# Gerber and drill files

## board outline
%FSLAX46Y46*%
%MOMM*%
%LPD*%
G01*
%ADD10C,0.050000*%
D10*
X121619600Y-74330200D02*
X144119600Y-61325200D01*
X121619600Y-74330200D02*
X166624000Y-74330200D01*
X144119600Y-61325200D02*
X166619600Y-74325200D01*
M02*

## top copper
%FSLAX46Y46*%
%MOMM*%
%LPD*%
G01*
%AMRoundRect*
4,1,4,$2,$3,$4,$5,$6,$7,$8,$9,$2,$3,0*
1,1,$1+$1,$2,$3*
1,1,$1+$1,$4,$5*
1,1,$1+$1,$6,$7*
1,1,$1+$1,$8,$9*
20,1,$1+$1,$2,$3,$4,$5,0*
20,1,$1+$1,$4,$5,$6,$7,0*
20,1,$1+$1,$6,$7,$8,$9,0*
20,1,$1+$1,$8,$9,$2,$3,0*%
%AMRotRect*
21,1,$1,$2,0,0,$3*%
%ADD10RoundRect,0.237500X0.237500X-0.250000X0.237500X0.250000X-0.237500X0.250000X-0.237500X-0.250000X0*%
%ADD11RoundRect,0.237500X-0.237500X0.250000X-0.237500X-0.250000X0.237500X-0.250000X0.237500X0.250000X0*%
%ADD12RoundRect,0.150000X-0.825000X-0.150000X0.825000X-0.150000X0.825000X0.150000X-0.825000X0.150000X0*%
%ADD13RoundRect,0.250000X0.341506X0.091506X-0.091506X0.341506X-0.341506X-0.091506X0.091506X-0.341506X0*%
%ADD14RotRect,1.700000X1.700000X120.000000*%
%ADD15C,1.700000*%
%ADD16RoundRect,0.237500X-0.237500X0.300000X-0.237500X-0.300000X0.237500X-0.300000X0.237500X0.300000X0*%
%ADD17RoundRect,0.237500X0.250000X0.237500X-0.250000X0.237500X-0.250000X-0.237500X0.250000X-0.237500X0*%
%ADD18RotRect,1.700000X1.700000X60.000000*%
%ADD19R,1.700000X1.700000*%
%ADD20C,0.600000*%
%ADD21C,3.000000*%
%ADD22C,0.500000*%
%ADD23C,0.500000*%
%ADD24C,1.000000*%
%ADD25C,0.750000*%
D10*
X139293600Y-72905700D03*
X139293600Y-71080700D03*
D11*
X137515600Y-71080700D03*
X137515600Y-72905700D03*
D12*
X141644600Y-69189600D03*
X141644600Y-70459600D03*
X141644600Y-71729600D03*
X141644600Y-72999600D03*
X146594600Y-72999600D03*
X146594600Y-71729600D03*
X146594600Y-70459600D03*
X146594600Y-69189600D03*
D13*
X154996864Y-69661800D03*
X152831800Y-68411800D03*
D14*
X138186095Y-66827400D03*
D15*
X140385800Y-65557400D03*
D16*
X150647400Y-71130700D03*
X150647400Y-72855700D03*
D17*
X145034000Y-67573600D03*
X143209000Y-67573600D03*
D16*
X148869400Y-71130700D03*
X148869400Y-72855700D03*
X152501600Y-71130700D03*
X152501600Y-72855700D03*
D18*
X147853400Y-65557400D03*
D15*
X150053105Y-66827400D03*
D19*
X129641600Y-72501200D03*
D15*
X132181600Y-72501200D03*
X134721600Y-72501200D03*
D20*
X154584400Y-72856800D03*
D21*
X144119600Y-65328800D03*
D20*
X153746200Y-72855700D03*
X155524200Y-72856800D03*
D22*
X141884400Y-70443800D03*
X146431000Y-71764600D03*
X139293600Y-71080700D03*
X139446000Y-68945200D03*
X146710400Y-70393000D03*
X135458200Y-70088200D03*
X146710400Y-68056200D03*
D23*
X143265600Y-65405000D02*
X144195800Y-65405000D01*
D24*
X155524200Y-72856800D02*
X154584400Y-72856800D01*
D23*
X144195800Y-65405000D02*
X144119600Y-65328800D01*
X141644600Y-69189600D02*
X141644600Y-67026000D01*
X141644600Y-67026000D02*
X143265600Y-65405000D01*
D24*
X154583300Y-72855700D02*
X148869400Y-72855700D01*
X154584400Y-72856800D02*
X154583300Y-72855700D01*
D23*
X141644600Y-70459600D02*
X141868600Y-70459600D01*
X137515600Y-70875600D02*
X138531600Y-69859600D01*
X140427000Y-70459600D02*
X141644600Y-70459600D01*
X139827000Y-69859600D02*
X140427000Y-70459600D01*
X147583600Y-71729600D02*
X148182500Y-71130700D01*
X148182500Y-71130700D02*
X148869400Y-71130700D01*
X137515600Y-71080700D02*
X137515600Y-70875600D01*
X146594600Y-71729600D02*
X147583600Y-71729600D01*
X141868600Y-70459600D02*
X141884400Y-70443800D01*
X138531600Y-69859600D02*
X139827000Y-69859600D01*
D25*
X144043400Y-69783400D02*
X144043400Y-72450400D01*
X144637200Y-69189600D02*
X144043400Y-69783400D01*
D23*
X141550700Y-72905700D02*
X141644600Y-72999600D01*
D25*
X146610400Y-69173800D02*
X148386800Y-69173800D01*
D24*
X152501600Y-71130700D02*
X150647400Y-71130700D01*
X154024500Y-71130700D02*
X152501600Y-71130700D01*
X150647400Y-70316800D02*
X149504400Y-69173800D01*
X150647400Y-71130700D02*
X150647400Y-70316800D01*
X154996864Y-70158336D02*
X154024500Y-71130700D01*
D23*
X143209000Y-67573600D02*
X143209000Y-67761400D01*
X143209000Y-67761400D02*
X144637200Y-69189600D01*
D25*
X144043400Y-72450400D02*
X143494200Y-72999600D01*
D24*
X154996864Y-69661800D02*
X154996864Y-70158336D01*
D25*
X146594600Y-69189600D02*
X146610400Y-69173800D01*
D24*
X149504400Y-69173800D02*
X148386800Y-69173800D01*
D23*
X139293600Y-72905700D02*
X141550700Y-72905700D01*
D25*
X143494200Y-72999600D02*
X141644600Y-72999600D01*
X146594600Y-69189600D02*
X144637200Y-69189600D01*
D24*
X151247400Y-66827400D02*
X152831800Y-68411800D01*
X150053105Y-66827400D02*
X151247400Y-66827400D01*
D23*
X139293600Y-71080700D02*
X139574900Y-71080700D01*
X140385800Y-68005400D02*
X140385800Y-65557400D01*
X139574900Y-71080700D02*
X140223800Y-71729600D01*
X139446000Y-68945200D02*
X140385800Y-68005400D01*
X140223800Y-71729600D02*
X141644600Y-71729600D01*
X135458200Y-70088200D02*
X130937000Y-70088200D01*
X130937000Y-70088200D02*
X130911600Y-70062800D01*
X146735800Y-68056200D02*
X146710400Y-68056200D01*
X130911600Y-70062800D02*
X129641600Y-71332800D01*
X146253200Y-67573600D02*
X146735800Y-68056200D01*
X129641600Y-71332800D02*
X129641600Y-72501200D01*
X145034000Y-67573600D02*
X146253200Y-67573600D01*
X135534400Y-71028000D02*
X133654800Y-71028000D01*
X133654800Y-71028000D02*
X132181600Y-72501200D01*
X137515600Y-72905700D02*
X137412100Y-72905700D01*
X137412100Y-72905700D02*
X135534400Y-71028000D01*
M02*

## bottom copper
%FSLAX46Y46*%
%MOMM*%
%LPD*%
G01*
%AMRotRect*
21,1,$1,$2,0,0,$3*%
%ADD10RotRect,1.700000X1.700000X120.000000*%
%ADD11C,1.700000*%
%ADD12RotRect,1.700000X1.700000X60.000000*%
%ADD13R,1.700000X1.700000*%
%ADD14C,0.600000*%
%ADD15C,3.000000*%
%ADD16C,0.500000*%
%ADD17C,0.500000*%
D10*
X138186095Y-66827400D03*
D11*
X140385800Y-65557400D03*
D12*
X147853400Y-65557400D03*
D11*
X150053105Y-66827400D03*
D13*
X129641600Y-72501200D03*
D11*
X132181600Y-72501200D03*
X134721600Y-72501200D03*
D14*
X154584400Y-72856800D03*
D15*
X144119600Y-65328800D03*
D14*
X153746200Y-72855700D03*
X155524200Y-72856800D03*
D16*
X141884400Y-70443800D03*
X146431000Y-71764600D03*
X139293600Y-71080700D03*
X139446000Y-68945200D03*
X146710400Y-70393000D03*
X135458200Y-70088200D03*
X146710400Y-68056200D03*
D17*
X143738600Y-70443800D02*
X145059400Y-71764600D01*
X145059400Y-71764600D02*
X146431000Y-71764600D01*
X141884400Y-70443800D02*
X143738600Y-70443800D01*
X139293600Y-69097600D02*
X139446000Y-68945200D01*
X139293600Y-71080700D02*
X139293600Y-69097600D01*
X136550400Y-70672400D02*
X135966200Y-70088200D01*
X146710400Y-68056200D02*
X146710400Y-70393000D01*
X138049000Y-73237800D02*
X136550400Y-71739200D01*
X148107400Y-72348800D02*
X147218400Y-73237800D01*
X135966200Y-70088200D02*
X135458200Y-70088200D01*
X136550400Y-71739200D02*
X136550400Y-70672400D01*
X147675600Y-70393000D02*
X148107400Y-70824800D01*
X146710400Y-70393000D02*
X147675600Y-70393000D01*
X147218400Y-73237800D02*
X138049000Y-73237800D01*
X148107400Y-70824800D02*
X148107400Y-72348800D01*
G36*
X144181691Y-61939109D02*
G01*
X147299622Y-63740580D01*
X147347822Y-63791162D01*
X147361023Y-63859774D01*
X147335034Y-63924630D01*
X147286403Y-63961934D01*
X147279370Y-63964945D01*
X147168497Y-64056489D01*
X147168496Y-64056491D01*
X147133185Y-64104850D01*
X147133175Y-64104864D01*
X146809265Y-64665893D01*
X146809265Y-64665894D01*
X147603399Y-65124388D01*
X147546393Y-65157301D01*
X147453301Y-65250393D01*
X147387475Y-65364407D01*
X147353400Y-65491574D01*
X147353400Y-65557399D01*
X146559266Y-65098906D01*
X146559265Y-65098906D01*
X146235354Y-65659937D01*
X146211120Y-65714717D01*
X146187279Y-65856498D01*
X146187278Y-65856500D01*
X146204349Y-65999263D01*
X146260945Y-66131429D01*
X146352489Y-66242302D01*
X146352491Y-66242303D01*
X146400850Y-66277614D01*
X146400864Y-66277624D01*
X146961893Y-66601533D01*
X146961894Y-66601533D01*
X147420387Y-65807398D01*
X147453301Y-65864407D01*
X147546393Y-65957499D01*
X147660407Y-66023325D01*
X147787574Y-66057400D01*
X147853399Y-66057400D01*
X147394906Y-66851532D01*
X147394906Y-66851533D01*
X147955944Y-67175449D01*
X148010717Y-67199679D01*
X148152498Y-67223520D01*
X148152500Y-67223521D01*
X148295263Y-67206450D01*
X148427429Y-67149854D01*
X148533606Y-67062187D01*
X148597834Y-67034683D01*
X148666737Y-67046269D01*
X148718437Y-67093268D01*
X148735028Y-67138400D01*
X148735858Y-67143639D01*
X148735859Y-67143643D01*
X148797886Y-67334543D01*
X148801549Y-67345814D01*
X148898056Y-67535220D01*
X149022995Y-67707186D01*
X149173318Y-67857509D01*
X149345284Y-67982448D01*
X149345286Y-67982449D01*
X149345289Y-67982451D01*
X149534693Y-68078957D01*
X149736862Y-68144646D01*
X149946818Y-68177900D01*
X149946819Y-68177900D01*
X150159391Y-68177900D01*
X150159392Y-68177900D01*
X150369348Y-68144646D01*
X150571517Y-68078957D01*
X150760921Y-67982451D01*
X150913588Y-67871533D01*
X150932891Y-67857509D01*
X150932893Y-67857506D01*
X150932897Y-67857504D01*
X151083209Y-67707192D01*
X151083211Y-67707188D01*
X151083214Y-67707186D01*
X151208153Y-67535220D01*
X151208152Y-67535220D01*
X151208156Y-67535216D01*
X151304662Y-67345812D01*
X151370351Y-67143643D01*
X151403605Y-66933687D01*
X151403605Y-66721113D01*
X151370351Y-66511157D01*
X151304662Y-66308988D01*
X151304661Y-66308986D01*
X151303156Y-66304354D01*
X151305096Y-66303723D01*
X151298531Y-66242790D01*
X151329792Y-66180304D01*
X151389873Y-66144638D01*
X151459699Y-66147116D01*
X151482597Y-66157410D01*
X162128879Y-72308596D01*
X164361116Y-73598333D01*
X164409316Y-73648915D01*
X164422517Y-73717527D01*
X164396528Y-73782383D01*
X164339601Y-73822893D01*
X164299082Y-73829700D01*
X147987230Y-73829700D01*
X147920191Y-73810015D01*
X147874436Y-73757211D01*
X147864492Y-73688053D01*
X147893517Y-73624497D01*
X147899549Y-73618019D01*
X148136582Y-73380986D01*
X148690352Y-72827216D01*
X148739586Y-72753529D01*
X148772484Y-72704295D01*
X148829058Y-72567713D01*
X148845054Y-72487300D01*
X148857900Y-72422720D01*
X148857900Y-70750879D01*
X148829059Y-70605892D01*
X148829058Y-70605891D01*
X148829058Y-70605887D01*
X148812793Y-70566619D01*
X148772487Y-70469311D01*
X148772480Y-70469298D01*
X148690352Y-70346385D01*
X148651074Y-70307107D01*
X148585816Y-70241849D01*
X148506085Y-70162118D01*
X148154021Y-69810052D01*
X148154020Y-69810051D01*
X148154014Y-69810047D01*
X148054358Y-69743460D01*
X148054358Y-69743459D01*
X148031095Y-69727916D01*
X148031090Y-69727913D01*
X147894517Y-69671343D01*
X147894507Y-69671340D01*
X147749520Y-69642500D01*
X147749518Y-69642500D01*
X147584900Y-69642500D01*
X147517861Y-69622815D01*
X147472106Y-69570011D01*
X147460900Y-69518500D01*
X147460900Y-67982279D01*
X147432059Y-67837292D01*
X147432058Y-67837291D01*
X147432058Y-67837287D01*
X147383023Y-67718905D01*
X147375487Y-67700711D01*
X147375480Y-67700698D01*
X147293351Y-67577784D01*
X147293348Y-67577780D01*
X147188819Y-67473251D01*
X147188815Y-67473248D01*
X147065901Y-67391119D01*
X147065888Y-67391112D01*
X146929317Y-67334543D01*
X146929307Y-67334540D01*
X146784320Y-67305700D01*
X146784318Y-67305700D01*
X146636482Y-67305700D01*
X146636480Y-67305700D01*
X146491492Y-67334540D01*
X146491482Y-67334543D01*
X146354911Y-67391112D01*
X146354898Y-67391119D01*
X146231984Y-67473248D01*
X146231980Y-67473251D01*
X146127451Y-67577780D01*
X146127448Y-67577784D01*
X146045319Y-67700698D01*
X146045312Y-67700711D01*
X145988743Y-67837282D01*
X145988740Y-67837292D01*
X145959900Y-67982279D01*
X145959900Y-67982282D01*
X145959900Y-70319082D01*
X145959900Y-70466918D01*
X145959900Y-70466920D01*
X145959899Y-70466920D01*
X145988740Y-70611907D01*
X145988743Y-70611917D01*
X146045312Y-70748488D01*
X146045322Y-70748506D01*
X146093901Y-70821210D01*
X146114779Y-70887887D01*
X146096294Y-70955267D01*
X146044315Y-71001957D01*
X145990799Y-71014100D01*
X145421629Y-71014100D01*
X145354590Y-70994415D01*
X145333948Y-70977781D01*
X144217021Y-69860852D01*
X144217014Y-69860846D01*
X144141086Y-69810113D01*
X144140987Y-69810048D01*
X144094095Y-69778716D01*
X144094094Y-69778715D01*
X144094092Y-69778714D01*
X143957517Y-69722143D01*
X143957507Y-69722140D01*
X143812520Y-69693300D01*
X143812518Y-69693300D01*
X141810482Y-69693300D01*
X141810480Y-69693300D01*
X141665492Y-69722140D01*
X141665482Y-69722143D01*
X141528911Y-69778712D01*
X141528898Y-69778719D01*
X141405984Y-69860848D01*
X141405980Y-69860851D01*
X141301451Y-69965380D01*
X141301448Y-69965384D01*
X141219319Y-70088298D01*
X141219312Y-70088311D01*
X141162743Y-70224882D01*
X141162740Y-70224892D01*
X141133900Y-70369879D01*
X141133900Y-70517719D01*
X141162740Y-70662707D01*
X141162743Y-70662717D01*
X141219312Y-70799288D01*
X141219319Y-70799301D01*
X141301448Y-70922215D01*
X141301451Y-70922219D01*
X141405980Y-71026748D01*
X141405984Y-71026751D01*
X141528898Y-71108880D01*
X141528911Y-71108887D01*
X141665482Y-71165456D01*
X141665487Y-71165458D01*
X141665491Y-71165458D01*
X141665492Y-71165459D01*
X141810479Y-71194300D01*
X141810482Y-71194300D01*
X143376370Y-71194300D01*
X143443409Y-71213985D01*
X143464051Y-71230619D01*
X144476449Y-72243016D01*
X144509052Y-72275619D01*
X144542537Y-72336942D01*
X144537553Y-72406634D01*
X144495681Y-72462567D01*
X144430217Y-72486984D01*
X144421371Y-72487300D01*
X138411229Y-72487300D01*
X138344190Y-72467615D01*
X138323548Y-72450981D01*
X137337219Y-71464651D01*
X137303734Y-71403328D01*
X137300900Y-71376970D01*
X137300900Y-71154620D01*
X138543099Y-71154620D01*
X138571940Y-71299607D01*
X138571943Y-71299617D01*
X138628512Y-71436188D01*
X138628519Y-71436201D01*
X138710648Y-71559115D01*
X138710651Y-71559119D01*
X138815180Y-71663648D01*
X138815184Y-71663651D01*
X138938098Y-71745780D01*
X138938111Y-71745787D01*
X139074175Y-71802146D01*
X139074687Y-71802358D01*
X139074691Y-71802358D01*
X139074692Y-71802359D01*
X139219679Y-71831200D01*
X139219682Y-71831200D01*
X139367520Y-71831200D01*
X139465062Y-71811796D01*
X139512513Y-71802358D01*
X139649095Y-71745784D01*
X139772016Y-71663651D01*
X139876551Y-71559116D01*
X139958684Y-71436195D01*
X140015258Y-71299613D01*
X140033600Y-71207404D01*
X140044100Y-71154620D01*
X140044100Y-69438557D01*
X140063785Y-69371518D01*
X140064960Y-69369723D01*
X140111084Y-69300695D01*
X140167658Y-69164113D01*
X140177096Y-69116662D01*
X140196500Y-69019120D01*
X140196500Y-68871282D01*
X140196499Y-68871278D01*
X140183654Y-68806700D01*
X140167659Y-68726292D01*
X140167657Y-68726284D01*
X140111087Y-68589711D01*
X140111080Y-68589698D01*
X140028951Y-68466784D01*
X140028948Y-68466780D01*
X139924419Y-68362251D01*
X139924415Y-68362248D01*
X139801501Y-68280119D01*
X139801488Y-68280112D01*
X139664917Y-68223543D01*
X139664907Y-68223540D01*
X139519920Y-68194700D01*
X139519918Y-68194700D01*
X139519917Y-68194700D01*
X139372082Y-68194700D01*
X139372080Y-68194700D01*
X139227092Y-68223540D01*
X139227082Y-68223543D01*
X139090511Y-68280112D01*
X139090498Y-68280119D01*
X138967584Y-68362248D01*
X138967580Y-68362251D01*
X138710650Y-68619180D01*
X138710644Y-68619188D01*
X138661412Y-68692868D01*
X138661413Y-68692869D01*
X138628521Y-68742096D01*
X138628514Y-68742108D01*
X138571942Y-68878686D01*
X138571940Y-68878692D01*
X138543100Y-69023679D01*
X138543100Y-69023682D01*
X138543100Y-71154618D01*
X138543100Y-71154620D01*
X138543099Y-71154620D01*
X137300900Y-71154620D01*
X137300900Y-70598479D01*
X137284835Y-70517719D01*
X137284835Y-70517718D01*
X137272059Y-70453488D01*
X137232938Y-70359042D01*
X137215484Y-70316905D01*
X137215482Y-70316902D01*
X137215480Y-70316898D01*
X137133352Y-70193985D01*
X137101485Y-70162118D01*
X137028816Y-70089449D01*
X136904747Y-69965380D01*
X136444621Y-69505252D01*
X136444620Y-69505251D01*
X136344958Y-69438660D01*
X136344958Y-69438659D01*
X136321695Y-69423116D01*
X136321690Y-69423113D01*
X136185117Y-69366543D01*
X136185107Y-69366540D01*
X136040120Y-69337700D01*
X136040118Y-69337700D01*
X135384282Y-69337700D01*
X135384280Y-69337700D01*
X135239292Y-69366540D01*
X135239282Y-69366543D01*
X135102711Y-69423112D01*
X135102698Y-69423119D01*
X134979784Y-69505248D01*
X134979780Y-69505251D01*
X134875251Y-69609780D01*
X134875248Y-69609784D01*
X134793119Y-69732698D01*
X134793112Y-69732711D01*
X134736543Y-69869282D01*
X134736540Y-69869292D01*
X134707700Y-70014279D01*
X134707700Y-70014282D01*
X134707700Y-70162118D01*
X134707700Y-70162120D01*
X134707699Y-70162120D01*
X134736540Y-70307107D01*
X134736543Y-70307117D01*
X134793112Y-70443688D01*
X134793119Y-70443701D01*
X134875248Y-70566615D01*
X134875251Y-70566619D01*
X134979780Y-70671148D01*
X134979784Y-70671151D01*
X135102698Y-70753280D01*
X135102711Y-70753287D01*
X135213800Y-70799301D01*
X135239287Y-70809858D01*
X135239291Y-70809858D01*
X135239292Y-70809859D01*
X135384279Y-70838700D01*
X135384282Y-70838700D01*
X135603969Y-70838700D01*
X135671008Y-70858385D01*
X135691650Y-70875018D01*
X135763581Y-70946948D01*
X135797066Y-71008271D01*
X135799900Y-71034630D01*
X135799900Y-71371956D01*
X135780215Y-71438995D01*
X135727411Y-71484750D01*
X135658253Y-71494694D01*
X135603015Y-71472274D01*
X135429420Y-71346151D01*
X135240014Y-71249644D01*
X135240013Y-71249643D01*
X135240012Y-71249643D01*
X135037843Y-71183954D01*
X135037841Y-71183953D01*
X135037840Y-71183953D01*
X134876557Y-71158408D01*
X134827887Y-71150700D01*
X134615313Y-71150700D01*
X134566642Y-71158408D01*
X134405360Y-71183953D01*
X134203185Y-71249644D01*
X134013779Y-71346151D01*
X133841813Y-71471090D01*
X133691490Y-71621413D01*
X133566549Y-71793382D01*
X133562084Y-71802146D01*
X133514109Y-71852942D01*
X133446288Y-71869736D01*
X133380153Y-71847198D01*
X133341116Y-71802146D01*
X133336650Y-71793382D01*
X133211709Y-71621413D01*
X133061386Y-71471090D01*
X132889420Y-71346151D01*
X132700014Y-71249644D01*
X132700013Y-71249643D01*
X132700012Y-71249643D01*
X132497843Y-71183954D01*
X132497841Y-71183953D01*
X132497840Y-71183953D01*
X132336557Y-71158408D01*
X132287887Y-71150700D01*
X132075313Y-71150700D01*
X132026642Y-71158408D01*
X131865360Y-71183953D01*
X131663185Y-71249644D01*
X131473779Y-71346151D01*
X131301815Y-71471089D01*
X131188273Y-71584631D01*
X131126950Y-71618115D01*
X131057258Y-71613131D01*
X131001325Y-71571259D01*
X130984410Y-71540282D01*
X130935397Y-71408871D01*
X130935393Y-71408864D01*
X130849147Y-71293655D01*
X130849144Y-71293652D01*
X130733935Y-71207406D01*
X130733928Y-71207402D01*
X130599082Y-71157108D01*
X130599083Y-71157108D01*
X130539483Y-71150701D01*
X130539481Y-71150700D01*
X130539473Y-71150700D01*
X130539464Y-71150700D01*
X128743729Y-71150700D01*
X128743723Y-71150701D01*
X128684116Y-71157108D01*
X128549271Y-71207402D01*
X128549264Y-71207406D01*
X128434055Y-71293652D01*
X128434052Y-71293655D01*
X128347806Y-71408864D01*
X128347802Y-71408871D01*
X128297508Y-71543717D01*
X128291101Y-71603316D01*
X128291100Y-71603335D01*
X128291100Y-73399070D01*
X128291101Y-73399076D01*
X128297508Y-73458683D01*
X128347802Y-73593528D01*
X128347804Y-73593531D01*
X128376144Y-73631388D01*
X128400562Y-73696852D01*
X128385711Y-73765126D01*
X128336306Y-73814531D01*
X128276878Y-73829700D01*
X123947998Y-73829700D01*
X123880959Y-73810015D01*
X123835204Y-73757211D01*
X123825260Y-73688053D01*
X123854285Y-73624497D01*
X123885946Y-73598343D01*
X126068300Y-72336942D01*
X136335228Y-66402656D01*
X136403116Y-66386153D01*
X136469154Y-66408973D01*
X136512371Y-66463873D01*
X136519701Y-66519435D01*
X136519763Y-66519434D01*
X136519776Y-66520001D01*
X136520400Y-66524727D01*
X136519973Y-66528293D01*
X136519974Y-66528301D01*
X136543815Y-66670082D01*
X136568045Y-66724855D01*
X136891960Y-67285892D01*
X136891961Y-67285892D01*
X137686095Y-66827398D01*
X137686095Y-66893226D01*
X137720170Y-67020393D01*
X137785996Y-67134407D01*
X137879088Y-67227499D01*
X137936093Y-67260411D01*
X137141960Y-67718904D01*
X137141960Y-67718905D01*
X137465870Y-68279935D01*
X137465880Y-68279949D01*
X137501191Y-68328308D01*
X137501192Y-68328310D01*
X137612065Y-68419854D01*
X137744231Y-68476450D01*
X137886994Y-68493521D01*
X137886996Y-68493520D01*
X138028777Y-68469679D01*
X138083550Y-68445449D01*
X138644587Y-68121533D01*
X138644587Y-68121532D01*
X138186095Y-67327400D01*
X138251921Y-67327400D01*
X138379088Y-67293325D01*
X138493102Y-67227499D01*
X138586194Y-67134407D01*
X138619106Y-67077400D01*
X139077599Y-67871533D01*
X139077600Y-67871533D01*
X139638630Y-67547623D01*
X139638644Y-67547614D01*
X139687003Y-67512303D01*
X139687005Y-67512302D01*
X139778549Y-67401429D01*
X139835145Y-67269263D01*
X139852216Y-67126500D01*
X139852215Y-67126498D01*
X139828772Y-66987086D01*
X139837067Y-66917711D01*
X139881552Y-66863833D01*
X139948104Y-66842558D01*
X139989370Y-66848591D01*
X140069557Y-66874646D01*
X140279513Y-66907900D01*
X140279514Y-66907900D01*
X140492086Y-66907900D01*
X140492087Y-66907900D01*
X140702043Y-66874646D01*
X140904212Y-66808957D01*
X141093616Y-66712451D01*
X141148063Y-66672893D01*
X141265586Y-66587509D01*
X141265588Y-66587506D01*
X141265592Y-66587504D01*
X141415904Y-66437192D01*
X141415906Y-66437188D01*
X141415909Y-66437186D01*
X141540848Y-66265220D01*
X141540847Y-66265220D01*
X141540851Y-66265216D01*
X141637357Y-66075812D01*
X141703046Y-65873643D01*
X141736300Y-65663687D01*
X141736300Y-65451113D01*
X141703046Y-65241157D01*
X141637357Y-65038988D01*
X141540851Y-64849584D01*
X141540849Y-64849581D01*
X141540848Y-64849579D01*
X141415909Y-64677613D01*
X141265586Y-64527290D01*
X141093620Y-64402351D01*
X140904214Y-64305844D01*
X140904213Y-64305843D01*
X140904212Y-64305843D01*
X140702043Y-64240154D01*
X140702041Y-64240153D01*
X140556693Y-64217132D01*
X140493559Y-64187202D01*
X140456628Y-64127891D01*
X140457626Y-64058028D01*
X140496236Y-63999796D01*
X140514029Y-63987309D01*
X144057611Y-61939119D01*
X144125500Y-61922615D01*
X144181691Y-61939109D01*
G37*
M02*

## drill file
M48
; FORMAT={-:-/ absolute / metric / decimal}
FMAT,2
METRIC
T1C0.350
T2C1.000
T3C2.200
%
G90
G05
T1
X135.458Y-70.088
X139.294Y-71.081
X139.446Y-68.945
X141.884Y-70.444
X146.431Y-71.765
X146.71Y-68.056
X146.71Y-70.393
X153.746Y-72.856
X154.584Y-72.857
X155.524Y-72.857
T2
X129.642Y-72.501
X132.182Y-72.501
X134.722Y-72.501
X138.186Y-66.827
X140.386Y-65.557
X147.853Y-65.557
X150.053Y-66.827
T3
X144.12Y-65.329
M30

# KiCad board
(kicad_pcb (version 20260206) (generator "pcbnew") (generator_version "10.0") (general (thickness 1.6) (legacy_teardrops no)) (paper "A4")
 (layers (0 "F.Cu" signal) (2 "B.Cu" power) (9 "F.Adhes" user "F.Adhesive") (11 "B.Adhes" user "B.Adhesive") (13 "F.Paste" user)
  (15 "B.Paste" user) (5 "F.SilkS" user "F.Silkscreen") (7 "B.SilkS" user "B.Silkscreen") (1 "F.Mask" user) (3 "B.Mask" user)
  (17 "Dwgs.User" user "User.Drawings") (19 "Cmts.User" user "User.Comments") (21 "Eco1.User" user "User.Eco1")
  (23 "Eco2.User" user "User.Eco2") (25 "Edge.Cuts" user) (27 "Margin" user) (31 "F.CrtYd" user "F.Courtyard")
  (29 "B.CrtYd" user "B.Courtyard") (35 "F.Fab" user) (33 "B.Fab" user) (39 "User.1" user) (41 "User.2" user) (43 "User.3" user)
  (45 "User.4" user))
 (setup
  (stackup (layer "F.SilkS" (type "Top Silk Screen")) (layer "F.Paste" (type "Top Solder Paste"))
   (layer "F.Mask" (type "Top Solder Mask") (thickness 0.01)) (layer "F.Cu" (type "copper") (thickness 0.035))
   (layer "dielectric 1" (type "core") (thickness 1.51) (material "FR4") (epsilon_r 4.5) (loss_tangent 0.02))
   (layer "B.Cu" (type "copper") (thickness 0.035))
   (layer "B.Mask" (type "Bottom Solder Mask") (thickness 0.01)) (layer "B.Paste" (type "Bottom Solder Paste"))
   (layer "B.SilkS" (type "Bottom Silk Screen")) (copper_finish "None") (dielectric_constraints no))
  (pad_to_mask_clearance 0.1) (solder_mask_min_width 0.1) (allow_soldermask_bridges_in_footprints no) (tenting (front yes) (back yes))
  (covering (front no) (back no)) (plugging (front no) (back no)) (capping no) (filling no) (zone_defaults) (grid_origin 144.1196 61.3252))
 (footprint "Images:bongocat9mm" (layer "F.Cu") (at 158.0388 72.806)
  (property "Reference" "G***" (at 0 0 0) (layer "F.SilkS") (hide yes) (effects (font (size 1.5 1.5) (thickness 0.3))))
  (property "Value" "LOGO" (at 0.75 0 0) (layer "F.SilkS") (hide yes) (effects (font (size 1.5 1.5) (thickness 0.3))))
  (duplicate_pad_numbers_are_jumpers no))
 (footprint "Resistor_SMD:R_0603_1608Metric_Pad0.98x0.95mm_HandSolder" (layer "F.Cu") (at 139.2936 71.9932 90)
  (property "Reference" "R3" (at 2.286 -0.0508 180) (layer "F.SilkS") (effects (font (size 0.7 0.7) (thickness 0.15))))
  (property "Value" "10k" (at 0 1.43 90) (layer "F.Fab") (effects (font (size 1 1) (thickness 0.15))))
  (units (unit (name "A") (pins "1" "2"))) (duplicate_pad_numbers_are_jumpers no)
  (pad "1" smd roundrect (at -0.9125 0 90) (size 0.975 0.95) (layers "F.Cu" "F.Mask" "F.Paste") (roundrect_rratio 0.25) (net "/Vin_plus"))
  (pad "2" smd roundrect (at 0.9125 0 90) (size 0.975 0.95) (layers "F.Cu" "F.Mask" "F.Paste") (roundrect_rratio 0.25) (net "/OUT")))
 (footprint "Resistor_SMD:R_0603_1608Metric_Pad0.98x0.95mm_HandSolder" (layer "F.Cu") (at 137.5156 71.9932 -90)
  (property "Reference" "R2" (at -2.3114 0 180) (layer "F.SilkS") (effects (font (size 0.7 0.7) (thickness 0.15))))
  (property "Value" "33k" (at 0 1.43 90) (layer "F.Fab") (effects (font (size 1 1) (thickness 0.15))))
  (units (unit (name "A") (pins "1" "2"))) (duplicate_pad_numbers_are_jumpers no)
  (pad "1" smd roundrect (at -0.9125 0 270) (size 0.975 0.95) (layers "F.Cu" "F.Mask" "F.Paste") (roundrect_rratio 0.25)
   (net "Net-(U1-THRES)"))
  (pad "2" smd roundrect (at 0.9125 0 270) (size 0.975 0.95) (layers "F.Cu" "F.Mask" "F.Paste") (roundrect_rratio 0.25)
   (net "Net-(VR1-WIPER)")))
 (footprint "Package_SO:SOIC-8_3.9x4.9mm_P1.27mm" (layer "F.Cu") (at 144.1196 71.0946)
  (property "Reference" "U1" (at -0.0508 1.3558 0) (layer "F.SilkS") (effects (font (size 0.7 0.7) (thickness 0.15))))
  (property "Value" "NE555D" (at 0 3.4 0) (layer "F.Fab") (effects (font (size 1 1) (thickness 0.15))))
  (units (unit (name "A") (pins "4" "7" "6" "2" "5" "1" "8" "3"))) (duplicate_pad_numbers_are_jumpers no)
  (pad "1" smd roundrect (at -2.475 -1.905) (size 1.95 0.6) (layers "F.Cu" "F.Mask" "F.Paste") (roundrect_rratio 0.25) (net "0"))
  (pad "2" smd roundrect (at -2.475 -0.635) (size 1.95 0.6) (layers "F.Cu" "F.Mask" "F.Paste") (roundrect_rratio 0.25)
   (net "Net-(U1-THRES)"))
  (pad "3" smd roundrect (at -2.475 0.635) (size 1.95 0.6) (layers "F.Cu" "F.Mask" "F.Paste") (roundrect_rratio 0.25) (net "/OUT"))
  (pad "4" smd roundrect (at -2.475 1.905) (size 1.95 0.6) (layers "F.Cu" "F.Mask" "F.Paste") (roundrect_rratio 0.25) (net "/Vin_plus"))
  (pad "5" smd roundrect (at 2.475 1.905) (size 1.95 0.6) (layers "F.Cu" "F.Mask" "F.Paste") (roundrect_rratio 0.25)
   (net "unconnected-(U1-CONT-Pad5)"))
  (pad "6" smd roundrect (at 2.475 0.635) (size 1.95 0.6) (layers "F.Cu" "F.Mask" "F.Paste") (roundrect_rratio 0.25) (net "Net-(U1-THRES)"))
  (pad "7" smd roundrect (at 2.475 -0.635) (size 1.95 0.6) (layers "F.Cu" "F.Mask" "F.Paste") (roundrect_rratio 0.25) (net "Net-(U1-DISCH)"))
  (pad "8" smd roundrect (at 2.475 -1.905) (size 1.95 0.6) (layers "F.Cu" "F.Mask" "F.Paste") (roundrect_rratio 0.25) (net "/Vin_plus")))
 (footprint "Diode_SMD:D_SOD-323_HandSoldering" (layer "F.Cu") (at 153.914332 69.0368 150)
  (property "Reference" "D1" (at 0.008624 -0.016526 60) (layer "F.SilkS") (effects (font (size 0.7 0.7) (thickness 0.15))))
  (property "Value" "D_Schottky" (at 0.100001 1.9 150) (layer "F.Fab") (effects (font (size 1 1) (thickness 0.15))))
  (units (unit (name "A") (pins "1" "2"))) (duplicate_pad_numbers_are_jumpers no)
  (pad "1" smd roundrect (at -1.25 0 150) (size 1 1) (layers "F.Cu" "F.Mask" "F.Paste") (roundrect_rratio 0.25) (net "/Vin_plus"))
  (pad "2" smd roundrect (at 1.25 0 150) (size 1 1) (layers "F.Cu" "F.Mask" "F.Paste") (roundrect_rratio 0.25) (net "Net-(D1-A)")))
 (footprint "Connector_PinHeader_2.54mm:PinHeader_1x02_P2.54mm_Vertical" (layer "F.Cu") (at 138.186095 66.8274 120)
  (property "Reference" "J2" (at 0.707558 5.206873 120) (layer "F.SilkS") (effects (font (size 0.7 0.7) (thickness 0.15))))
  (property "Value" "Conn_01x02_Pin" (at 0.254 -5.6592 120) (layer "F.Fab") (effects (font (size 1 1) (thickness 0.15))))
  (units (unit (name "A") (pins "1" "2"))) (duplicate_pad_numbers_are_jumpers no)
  (pad "1" thru_hole rect (at 0 0 120) (size 1.7 1.7) (drill 1) (layers "*.Cu" "*.Mask") (remove_unused_layers no) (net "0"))
  (pad "2" thru_hole circle (at 0 2.54 120) (size 1.7 1.7) (drill 1) (layers "*.Cu" "*.Mask") (remove_unused_layers no) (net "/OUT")))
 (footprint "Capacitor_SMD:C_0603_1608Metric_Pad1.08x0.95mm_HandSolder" (layer "F.Cu") (at 150.6474 71.9932 -90)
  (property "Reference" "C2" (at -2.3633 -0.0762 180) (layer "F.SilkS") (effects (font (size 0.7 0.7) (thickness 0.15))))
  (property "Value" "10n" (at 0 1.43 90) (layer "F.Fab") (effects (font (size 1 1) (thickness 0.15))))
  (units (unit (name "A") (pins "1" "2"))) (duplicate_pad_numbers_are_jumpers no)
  (pad "1" smd roundrect (at -0.8625 0 270) (size 1.075 0.95) (layers "F.Cu" "F.Mask" "F.Paste") (roundrect_rratio 0.25) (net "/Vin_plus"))
  (pad "2" smd roundrect (at 0.8625 0 270) (size 1.075 0.95) (layers "F.Cu" "F.Mask" "F.Paste") (roundrect_rratio 0.25) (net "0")))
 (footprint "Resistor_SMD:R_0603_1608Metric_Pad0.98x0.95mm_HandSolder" (layer "F.Cu") (at 144.1215 67.5736 180)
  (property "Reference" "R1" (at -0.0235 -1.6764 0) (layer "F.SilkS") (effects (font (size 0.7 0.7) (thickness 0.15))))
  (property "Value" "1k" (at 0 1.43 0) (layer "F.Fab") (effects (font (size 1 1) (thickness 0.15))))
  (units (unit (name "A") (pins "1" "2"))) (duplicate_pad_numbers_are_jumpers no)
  (pad "1" smd roundrect (at -0.9125 0 180) (size 0.975 0.95) (layers "F.Cu" "F.Mask" "F.Paste") (roundrect_rratio 0.25)
   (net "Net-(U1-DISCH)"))
  (pad "2" smd roundrect (at 0.9125 0 180) (size 0.975 0.95) (layers "F.Cu" "F.Mask" "F.Paste") (roundrect_rratio 0.25) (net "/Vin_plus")))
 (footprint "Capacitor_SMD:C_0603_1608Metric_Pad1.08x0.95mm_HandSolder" (layer "F.Cu") (at 148.8694 71.9932 -90)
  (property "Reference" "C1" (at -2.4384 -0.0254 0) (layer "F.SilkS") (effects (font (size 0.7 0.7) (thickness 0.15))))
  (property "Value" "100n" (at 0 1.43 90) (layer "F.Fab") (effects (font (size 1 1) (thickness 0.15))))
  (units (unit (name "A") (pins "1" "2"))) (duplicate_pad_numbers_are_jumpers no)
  (pad "1" smd roundrect (at -0.8625 0 270) (size 1.075 0.95) (layers "F.Cu" "F.Mask" "F.Paste") (roundrect_rratio 0.25)
   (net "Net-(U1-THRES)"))
  (pad "2" smd roundrect (at 0.8625 0 270) (size 1.075 0.95) (layers "F.Cu" "F.Mask" "F.Paste") (roundrect_rratio 0.25) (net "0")))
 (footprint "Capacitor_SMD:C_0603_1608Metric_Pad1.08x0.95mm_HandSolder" (layer "F.Cu") (at 152.5016 71.9932 -90)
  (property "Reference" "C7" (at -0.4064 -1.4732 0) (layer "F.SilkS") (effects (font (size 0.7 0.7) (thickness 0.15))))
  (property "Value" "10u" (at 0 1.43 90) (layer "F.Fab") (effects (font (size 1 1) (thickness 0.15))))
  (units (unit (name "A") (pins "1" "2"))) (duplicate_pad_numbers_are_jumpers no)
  (pad "1" smd roundrect (at -0.8625 0 270) (size 1.075 0.95) (layers "F.Cu" "F.Mask" "F.Paste") (roundrect_rratio 0.25) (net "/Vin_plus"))
  (pad "2" smd roundrect (at 0.8625 0 270) (size 1.075 0.95) (layers "F.Cu" "F.Mask" "F.Paste") (roundrect_rratio 0.25) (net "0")))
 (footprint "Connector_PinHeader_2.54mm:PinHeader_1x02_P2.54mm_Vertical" (layer "F.Cu") (at 147.8534 65.5574 60)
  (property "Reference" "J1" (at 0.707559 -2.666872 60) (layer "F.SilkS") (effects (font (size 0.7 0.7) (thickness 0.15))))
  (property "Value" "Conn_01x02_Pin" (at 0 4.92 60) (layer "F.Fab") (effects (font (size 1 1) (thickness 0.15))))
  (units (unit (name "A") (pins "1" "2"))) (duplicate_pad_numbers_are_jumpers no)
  (pad "1" thru_hole rect (at 0 0 60) (size 1.7 1.7) (drill 1) (layers "*.Cu" "*.Mask") (remove_unused_layers no) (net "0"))
  (pad "2" thru_hole circle (at 0 2.54 60) (size 1.7 1.7) (drill 1) (layers "*.Cu" "*.Mask") (remove_unused_layers no) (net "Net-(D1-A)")))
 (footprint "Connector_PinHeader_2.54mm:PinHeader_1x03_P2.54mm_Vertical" (layer "F.Cu") (at 129.6416 72.5012 90)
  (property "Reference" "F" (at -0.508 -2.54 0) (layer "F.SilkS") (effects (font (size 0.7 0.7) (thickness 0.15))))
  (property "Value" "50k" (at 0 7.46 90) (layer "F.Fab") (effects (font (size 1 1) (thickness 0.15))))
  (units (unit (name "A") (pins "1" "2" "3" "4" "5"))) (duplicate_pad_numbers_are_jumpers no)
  (pad "1" thru_hole rect (at 0 0 90) (size 1.7 1.7) (drill 1) (layers "*.Cu" "*.Mask") (remove_unused_layers no) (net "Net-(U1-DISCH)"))
  (pad "2" thru_hole circle (at 0 2.54 90) (size 1.7 1.7) (drill 1) (layers "*.Cu" "*.Mask") (remove_unused_layers no)
   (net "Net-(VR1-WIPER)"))
  (pad "3" thru_hole circle (at 0 5.08 90) (size 1.7 1.7) (drill 1) (layers "*.Cu" "*.Mask") (remove_unused_layers no)
   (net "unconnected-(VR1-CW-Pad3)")))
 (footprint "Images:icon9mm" (layer "B.Cu") (at 154.4066 71.1296 180)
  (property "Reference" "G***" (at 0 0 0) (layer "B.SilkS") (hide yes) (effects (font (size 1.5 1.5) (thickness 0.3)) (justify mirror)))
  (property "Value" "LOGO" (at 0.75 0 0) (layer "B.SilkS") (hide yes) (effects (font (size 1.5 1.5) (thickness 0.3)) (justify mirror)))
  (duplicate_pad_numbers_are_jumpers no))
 (gr_line (start 121.6196 74.3302) (end 144.1196 61.3252) (stroke (width 0.05) (type default)) (layer "Edge.Cuts"))
 (gr_line (start 121.6196 74.3302) (end 166.624 74.3302) (stroke (width 0.05) (type default)) (layer "Edge.Cuts"))
 (gr_line (start 144.1196 61.3252) (end 166.6196 74.3252) (stroke (width 0.05) (type default)) (layer "Edge.Cuts"))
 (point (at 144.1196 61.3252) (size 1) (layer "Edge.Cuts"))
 (segment (start 143.2656 65.405) (end 144.1958 65.405) (width 0.5) (layer "F.Cu") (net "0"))
 (segment (start 155.5242 72.8568) (end 154.5844 72.8568) (width 1) (layer "F.Cu") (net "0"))
 (segment (start 144.1958 65.405) (end 144.1196 65.3288) (width 0.5) (layer "F.Cu") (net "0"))
 (segment (start 141.6446 69.1896) (end 141.6446 67.026) (width 0.5) (layer "F.Cu") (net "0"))
 (segment (start 141.6446 67.026) (end 143.2656 65.405) (width 0.5) (layer "F.Cu") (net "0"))
 (segment (start 154.5833 72.8557) (end 148.8694 72.8557) (width 1) (layer "F.Cu") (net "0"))
 (segment (start 154.5844 72.8568) (end 154.5833 72.8557) (width 1) (layer "F.Cu") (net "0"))
 (via (at 154.5844 72.8568) (size 0.6) (drill 0.35) (layers "F.Cu" "B.Cu") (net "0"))
 (via (at 144.1196 65.3288) (size 3) (drill 2.2) (layers "F.Cu" "B.Cu") (free yes) (tenting (front no) (back no)) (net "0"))
 (via (at 153.7462 72.8557) (size 0.6) (drill 0.35) (layers "F.Cu" "B.Cu") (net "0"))
 (via (at 155.5242 72.8568) (size 0.6) (drill 0.35) (layers "F.Cu" "B.Cu") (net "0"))
 (segment (start 141.6446 70.4596) (end 141.8686 70.4596) (width 0.5) (layer "F.Cu") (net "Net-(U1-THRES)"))
 (segment (start 137.5156 70.8756) (end 138.5316 69.8596) (width 0.5) (layer "F.Cu") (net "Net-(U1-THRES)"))
 (segment (start 140.427 70.4596) (end 141.6446 70.4596) (width 0.5) (layer "F.Cu") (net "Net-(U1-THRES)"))
 (segment (start 139.827 69.8596) (end 140.427 70.4596) (width 0.5) (layer "F.Cu") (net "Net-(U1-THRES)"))
 (segment (start 147.5836 71.7296) (end 148.1825 71.1307) (width 0.5) (layer "F.Cu") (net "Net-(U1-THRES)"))
 (segment (start 148.1825 71.1307) (end 148.8694 71.1307) (width 0.5) (layer "F.Cu") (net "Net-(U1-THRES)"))
 (segment (start 137.5156 71.0807) (end 137.5156 70.8756) (width 0.5) (layer "F.Cu") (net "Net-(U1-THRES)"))
 (segment (start 146.5946 71.7296) (end 147.5836 71.7296) (width 0.5) (layer "F.Cu") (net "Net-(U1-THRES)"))
 (segment (start 141.8686 70.4596) (end 141.8844 70.4438) (width 0.5) (layer "F.Cu") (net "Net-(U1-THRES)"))
 (segment (start 138.5316 69.8596) (end 139.827 69.8596) (width 0.5) (layer "F.Cu") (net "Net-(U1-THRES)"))
 (via (at 141.8844 70.4438) (size 0.5) (drill 0.35) (layers "F.Cu" "B.Cu") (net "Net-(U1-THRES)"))
 (via (at 146.431 71.7646) (size 0.5) (drill 0.35) (layers "F.Cu" "B.Cu") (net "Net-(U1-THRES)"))
 (segment (start 143.7386 70.4438) (end 145.0594 71.7646) (width 0.5) (layer "B.Cu") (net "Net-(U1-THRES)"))
 (segment (start 145.0594 71.7646) (end 146.431 71.7646) (width 0.5) (layer "B.Cu") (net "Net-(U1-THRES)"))
 (segment (start 141.8844 70.4438) (end 143.7386 70.4438) (width 0.5) (layer "B.Cu") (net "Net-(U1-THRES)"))
 (segment (start 144.0434 69.7834) (end 144.0434 72.4504) (width 0.75) (layer "F.Cu") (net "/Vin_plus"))
 (segment (start 144.6372 69.1896) (end 144.0434 69.7834) (width 0.75) (layer "F.Cu") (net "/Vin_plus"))
 (segment (start 141.5507 72.9057) (end 141.6446 72.9996) (width 0.5) (layer "F.Cu") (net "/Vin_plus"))
 (segment (start 146.6104 69.1738) (end 148.3868 69.1738) (width 0.75) (layer "F.Cu") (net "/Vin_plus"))
 (segment (start 152.5016 71.1307) (end 150.6474 71.1307) (width 1) (layer "F.Cu") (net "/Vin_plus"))
 (segment (start 154.0245 71.1307) (end 152.5016 71.1307) (width 1) (layer "F.Cu") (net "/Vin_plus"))
 (segment (start 150.6474 70.3168) (end 149.5044 69.1738) (width 1) (layer "F.Cu") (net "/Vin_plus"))
 (segment (start 150.6474 71.1307) (end 150.6474 70.3168) (width 1) (layer "F.Cu") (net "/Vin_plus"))
 (segment (start 154.996864 70.158336) (end 154.0245 71.1307) (width 1) (layer "F.Cu") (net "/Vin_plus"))
 (segment (start 143.209 67.5736) (end 143.209 67.7614) (width 0.5) (layer "F.Cu") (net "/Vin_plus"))
 (segment (start 143.209 67.7614) (end 144.6372 69.1896) (width 0.5) (layer "F.Cu") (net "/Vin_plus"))
 (segment (start 144.0434 72.4504) (end 143.4942 72.9996) (width 0.75) (layer "F.Cu") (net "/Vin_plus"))
 (segment (start 154.996864 69.6618) (end 154.996864 70.158336) (width 1) (layer "F.Cu") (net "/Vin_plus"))
 (segment (start 146.5946 69.1896) (end 146.6104 69.1738) (width 0.75) (layer "F.Cu") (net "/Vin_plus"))
 (segment (start 149.5044 69.1738) (end 148.3868 69.1738) (width 1) (layer "F.Cu") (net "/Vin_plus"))
 (segment (start 139.2936 72.9057) (end 141.5507 72.9057) (width 0.5) (layer "F.Cu") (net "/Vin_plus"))
 (segment (start 143.4942 72.9996) (end 141.6446 72.9996) (width 0.75) (layer "F.Cu") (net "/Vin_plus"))
 (segment (start 146.5946 69.1896) (end 144.6372 69.1896) (width 0.75) (layer "F.Cu") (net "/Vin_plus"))
 (segment (start 151.2474 66.8274) (end 152.8318 68.4118) (width 1) (layer "F.Cu") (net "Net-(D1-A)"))
 (segment (start 150.053105 66.8274) (end 151.2474 66.8274) (width 1) (layer "F.Cu") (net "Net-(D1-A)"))
 (segment (start 139.2936 71.0807) (end 139.5749 71.0807) (width 0.5) (layer "F.Cu") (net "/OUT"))
 (segment (start 140.3858 68.0054) (end 140.3858 65.5574) (width 0.5) (layer "F.Cu") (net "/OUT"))
 (segment (start 139.5749 71.0807) (end 140.2238 71.7296) (width 0.5) (layer "F.Cu") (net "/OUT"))
 (segment (start 139.446 68.9452) (end 140.3858 68.0054) (width 0.5) (layer "F.Cu") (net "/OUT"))
 (segment (start 140.2238 71.7296) (end 141.6446 71.7296) (width 0.5) (layer "F.Cu") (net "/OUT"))
 (via (at 139.2936 71.0807) (size 0.5) (drill 0.35) (layers "F.Cu" "B.Cu") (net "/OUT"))
 (via (at 139.446 68.9452) (size 0.5) (drill 0.35) (layers "F.Cu" "B.Cu") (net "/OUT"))
 (segment (start 139.2936 69.0976) (end 139.446 68.9452) (width 0.5) (layer "B.Cu") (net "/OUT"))
 (segment (start 139.2936 71.0807) (end 139.2936 69.0976) (width 0.5) (layer "B.Cu") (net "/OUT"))
 (segment (start 135.4582 70.0882) (end 130.937 70.0882) (width 0.5) (layer "F.Cu") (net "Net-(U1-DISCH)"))
 (segment (start 130.937 70.0882) (end 130.9116 70.0628) (width 0.5) (layer "F.Cu") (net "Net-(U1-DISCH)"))
 (segment (start 146.7358 68.0562) (end 146.7104 68.0562) (width 0.5) (layer "F.Cu") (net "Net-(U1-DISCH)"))
 (segment (start 130.9116 70.0628) (end 129.6416 71.3328) (width 0.5) (layer "F.Cu") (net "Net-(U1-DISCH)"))
 (segment (start 146.2532 67.5736) (end 146.7358 68.0562) (width 0.5) (layer "F.Cu") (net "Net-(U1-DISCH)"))
 (segment (start 129.6416 71.3328) (end 129.6416 72.5012) (width 0.5) (layer "F.Cu") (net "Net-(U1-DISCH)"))
 (segment (start 145.034 67.5736) (end 146.2532 67.5736) (width 0.5) (layer "F.Cu") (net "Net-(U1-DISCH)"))
 (via (at 146.7104 70.393) (size 0.5) (drill 0.35) (layers "F.Cu" "B.Cu") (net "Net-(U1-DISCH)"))
 (via (at 135.4582 70.0882) (size 0.5) (drill 0.35) (layers "F.Cu" "B.Cu") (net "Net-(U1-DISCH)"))
 (via (at 146.7104 68.0562) (size 0.5) (drill 0.35) (layers "F.Cu" "B.Cu") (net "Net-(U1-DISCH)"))
 (segment (start 136.5504 70.6724) (end 135.9662 70.0882) (width 0.5) (layer "B.Cu") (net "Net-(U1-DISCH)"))
 (segment (start 146.7104 68.0562) (end 146.7104 70.393) (width 0.5) (layer "B.Cu") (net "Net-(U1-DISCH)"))
 (segment (start 138.049 73.2378) (end 136.5504 71.7392) (width 0.5) (layer "B.Cu") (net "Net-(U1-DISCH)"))
 (segment (start 148.1074 72.3488) (end 147.2184 73.2378) (width 0.5) (layer "B.Cu") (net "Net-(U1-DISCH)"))
 (segment (start 135.9662 70.0882) (end 135.4582 70.0882) (width 0.5) (layer "B.Cu") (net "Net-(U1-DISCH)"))
 (segment (start 136.5504 71.7392) (end 136.5504 70.6724) (width 0.5) (layer "B.Cu") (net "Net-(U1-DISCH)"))
 (segment (start 147.6756 70.393) (end 148.1074 70.8248) (width 0.5) (layer "B.Cu") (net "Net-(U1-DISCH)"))
 (segment (start 146.7104 70.393) (end 147.6756 70.393) (width 0.5) (layer "B.Cu") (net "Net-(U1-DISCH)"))
 (segment (start 147.2184 73.2378) (end 138.049 73.2378) (width 0.5) (layer "B.Cu") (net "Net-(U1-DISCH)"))
 (segment (start 148.1074 70.8248) (end 148.1074 72.3488) (width 0.5) (layer "B.Cu") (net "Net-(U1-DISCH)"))
 (segment (start 135.5344 71.028) (end 133.6548 71.028) (width 0.5) (layer "F.Cu") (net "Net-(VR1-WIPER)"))
 (segment (start 133.6548 71.028) (end 132.1816 72.5012) (width 0.5) (layer "F.Cu") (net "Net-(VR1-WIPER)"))
 (segment (start 137.5156 72.9057) (end 137.4121 72.9057) (width 0.5) (layer "F.Cu") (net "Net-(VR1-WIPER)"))
 (segment (start 137.4121 72.9057) (end 135.5344 71.028) (width 0.5) (layer "F.Cu") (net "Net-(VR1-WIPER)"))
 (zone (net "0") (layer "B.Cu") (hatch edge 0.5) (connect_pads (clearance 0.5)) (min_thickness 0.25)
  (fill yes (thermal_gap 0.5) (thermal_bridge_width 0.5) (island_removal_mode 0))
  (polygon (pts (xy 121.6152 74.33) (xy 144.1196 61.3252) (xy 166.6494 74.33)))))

